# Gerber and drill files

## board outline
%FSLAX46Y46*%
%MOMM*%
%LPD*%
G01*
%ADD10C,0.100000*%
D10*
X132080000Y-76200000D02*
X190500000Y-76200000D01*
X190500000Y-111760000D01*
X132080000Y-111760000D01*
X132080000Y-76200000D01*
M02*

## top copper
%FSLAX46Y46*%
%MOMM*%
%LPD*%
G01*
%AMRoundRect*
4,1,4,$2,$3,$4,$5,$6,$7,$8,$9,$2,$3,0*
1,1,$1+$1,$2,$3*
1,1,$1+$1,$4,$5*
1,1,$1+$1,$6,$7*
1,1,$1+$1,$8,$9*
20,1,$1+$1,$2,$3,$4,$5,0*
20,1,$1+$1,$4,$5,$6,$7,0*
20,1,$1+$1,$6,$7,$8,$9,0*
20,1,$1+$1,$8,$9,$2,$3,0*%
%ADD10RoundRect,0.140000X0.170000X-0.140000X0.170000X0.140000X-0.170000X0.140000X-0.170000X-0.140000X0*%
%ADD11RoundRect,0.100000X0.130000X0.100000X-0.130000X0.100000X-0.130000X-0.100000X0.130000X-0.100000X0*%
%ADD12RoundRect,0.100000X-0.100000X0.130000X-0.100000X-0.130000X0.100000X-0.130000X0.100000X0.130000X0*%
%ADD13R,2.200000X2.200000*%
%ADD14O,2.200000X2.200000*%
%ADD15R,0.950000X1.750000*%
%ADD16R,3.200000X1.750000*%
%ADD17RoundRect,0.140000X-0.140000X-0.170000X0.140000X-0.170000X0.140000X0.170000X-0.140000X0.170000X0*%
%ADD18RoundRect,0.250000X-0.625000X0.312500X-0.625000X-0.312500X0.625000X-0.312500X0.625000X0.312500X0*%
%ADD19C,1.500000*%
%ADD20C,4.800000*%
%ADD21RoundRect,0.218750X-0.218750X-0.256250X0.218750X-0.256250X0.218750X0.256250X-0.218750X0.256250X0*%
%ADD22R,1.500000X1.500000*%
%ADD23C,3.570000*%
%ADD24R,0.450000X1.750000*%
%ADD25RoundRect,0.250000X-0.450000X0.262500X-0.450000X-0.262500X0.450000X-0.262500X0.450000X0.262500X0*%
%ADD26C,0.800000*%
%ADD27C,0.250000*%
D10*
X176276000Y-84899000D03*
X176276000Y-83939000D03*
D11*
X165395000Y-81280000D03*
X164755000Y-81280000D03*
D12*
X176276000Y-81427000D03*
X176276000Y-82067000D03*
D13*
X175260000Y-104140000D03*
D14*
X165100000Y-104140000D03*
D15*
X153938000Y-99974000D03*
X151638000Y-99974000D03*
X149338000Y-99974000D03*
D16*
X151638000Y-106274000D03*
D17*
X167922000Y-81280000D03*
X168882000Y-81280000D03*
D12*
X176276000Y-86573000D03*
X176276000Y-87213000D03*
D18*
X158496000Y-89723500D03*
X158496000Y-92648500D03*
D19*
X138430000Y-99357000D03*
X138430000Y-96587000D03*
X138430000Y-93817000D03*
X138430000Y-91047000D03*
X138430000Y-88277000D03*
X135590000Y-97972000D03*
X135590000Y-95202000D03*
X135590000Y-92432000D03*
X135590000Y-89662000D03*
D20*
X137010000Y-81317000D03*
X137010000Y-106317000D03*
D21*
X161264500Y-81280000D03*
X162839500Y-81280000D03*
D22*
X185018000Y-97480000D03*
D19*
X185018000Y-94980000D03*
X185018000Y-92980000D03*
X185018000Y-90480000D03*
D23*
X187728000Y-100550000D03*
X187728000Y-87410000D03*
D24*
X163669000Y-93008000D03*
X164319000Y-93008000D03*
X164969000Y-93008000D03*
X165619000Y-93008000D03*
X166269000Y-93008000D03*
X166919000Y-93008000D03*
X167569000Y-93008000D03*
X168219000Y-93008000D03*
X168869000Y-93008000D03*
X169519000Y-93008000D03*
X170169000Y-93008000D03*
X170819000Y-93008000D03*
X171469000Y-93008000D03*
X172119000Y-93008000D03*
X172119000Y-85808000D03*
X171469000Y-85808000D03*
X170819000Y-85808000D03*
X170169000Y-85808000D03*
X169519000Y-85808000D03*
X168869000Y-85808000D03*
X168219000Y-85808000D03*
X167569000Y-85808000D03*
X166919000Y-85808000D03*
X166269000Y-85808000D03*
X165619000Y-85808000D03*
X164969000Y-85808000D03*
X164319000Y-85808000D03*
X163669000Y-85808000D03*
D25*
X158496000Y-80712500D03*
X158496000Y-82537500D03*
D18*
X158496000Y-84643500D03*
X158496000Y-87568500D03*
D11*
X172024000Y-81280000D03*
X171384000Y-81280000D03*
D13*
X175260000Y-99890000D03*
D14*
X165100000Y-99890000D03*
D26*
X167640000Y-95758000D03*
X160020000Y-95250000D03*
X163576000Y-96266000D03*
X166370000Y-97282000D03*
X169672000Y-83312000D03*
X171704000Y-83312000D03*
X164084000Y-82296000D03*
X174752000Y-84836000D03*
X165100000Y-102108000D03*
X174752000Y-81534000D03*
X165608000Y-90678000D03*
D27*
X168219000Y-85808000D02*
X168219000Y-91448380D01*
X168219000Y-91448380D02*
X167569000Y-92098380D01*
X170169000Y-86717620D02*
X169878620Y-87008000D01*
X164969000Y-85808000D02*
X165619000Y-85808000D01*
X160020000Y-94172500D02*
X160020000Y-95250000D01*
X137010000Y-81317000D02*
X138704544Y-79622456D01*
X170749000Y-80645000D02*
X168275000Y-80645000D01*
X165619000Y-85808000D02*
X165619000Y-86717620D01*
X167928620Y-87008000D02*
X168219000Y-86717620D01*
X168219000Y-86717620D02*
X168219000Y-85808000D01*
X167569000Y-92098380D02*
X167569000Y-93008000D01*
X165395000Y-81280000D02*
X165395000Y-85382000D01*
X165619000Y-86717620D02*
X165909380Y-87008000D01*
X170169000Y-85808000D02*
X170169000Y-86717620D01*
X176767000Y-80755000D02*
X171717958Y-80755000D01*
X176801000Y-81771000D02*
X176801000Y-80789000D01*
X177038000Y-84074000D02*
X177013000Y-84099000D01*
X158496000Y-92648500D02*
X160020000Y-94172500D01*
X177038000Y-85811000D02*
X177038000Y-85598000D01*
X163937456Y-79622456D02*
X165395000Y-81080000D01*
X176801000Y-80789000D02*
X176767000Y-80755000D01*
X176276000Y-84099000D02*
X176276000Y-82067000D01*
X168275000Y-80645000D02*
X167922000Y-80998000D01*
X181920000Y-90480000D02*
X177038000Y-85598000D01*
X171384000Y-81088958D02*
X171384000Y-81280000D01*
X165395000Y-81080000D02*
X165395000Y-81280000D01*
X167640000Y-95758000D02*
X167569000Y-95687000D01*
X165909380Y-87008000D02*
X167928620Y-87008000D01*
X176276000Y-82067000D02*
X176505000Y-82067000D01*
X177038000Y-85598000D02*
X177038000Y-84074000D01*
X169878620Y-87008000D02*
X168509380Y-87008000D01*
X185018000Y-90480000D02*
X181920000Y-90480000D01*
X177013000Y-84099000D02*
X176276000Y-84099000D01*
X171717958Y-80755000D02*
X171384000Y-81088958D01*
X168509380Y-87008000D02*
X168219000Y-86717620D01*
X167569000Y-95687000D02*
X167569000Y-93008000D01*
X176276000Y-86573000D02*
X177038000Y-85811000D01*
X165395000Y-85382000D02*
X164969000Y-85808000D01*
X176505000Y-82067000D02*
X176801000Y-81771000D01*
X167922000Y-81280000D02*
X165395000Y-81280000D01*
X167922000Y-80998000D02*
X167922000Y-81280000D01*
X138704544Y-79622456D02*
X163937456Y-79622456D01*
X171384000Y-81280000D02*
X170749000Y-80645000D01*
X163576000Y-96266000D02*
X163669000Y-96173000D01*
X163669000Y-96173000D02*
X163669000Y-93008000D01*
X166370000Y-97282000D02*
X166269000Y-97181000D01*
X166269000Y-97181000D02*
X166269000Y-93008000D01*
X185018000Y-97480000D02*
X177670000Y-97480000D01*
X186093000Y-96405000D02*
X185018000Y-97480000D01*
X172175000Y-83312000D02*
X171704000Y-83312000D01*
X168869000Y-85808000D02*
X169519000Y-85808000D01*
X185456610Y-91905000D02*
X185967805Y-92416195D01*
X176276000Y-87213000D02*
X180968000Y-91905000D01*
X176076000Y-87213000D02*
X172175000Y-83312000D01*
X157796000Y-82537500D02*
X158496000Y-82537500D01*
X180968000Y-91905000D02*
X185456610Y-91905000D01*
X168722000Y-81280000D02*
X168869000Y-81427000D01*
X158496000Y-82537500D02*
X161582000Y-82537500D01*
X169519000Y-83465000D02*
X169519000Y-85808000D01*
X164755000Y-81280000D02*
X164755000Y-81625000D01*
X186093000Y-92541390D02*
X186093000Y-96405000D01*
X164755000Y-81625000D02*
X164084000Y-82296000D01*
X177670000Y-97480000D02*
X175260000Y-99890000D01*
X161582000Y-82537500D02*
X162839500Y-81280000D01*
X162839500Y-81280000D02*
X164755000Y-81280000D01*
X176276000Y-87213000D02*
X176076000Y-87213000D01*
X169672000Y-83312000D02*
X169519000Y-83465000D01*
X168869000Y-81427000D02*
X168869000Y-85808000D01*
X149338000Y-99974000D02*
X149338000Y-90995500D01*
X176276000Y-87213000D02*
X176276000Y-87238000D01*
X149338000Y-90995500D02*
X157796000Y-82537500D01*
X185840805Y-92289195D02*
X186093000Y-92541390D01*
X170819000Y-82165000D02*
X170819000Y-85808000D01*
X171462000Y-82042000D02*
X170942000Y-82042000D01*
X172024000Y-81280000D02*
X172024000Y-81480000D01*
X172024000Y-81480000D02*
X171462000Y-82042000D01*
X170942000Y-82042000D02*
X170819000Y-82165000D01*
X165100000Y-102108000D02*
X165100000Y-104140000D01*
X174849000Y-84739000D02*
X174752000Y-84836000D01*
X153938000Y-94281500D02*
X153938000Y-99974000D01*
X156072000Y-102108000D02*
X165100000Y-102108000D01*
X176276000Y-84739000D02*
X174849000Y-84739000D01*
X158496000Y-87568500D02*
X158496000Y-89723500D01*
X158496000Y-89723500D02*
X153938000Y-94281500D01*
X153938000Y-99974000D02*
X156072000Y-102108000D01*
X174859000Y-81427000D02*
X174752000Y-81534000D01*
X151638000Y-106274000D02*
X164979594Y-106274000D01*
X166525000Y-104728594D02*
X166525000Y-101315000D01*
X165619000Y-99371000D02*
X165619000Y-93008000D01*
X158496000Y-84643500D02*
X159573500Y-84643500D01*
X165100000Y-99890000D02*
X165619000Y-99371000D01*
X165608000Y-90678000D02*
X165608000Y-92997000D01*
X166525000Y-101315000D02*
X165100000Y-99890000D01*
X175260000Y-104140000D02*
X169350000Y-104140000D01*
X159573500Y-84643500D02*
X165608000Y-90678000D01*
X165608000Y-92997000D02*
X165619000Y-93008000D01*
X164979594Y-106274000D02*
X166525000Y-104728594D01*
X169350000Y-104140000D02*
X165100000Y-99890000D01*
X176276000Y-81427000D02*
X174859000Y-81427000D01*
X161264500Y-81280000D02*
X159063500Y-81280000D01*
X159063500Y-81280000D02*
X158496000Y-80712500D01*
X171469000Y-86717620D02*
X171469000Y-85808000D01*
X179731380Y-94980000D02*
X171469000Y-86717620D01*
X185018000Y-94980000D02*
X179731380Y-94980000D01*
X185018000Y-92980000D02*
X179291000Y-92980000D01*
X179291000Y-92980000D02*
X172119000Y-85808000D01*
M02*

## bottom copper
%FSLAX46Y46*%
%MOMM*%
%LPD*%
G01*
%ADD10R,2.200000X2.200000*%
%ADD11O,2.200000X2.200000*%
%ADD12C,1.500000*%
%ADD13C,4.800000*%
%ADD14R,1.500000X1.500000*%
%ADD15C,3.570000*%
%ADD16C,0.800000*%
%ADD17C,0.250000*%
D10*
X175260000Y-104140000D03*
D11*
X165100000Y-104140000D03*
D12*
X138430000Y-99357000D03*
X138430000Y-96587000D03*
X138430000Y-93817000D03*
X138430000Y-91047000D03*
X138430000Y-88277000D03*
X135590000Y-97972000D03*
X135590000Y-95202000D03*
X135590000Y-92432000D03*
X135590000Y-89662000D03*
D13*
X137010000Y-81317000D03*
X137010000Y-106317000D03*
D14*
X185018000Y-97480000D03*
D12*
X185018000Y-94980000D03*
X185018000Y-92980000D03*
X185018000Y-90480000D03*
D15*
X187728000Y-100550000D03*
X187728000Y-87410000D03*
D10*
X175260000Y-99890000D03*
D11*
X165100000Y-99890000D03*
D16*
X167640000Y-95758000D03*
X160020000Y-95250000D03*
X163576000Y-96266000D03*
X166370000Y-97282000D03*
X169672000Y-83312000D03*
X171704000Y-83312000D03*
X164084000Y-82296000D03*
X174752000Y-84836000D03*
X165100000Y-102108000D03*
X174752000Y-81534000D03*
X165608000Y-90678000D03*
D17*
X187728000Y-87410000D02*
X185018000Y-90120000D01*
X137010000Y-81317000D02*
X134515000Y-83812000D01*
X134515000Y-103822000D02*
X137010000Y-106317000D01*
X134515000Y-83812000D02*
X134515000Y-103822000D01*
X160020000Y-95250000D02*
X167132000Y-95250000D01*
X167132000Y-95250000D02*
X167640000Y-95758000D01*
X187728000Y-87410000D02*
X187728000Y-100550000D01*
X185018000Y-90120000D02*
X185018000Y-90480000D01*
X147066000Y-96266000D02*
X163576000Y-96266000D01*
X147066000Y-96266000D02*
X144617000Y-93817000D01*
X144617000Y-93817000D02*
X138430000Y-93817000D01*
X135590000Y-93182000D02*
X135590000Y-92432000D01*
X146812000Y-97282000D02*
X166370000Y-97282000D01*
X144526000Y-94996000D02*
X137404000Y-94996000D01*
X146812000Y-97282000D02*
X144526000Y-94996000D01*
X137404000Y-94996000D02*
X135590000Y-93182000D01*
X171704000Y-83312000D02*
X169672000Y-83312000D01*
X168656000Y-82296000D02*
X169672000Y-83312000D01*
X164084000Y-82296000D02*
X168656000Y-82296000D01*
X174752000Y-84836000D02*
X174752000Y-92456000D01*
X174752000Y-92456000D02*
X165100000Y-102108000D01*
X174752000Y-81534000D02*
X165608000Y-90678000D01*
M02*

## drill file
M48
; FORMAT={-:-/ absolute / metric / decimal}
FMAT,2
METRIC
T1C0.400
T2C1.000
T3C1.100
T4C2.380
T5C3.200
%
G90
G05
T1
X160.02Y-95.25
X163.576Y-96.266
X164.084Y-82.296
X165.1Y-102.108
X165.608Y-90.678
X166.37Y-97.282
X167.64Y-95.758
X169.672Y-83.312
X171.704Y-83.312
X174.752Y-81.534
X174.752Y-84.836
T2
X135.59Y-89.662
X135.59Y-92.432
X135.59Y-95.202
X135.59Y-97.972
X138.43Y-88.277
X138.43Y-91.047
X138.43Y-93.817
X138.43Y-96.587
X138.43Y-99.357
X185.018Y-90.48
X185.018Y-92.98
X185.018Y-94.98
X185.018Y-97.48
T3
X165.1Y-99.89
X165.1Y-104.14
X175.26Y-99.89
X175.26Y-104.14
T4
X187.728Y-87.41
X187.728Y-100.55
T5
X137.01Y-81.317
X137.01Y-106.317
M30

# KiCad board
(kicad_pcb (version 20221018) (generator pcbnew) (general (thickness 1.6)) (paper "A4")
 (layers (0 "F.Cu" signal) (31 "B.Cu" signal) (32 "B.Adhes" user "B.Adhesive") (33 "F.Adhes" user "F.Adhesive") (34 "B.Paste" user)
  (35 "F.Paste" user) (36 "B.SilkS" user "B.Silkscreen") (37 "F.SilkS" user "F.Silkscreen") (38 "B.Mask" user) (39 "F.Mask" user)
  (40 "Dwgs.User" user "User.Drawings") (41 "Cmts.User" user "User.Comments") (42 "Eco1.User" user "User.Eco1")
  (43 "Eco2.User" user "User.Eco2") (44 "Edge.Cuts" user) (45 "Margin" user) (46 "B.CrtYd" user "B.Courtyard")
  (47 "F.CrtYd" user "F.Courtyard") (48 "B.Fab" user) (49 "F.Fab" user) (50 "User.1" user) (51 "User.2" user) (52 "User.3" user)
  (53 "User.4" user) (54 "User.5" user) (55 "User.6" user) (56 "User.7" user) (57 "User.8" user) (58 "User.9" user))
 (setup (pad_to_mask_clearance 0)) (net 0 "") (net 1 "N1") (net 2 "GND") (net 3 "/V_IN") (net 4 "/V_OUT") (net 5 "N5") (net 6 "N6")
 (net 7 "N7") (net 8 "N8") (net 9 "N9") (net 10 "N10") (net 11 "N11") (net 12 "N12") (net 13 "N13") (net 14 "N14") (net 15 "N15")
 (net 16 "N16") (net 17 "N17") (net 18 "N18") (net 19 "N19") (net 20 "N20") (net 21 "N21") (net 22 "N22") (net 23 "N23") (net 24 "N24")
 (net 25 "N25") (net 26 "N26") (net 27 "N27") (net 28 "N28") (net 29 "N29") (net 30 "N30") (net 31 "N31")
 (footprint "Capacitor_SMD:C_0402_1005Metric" (layer "F.Cu") (at 176.276 84.419 90)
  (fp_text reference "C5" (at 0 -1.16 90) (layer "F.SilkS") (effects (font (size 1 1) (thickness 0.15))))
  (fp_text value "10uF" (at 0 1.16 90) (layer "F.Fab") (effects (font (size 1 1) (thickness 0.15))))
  (pad "1" smd roundrect (at -0.48 0 90) (size 0.56 0.62) (layers "F.Cu" "F.Paste" "F.Mask") (roundrect_rratio 0.25) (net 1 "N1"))
  (pad "2" smd roundrect (at 0.48 0 90) (size 0.56 0.62) (layers "F.Cu" "F.Paste" "F.Mask") (roundrect_rratio 0.25) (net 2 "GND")))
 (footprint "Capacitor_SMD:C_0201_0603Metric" (layer "F.Cu") (at 165.075 81.28 180)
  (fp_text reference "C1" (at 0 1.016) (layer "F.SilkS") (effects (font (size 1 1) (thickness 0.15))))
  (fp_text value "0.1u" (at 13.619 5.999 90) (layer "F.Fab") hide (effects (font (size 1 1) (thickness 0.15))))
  (pad "" smd roundrect (at -0.345 0 180) (size 0.318 0.36) (layers "F.Paste") (roundrect_rratio 0.25))
  (pad "" smd roundrect (at 0.345 0 180) (size 0.318 0.36) (layers "F.Paste") (roundrect_rratio 0.25))
  (pad "1" smd roundrect (at -0.32 0 180) (size 0.46 0.4) (layers "F.Cu" "F.Mask") (roundrect_rratio 0.25) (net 2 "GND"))
  (pad "2" smd roundrect (at 0.32 0 180) (size 0.46 0.4) (layers "F.Cu" "F.Mask") (roundrect_rratio 0.25) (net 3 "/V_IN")))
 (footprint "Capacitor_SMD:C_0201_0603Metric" (layer "F.Cu") (at 176.276 81.747 -90)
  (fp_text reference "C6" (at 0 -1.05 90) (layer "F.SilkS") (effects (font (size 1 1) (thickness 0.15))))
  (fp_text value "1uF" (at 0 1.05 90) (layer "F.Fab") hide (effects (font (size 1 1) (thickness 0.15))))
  (pad "" smd roundrect (at -0.345 0 270) (size 0.318 0.36) (layers "F.Paste") (roundrect_rratio 0.25))
  (pad "" smd roundrect (at 0.345 0 270) (size 0.318 0.36) (layers "F.Paste") (roundrect_rratio 0.25))
  (pad "1" smd roundrect (at -0.32 0 270) (size 0.46 0.4) (layers "F.Cu" "F.Mask") (roundrect_rratio 0.25) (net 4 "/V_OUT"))
  (pad "2" smd roundrect (at 0.32 0 270) (size 0.46 0.4) (layers "F.Cu" "F.Mask") (roundrect_rratio 0.25) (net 2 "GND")))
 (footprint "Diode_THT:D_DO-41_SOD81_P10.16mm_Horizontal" (layer "F.Cu") (at 175.26 104.14 180)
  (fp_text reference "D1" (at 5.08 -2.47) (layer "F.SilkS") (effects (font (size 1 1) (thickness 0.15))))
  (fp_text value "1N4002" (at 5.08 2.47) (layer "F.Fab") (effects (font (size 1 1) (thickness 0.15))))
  (pad "1" thru_hole rect (at 0 0 180) (size 2.2 2.2) (drill 1.1) (layers "*.Cu" "*.Mask") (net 4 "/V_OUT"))
  (pad "2" thru_hole oval (at 10.16 0 180) (size 2.2 2.2) (drill 1.1) (layers "*.Cu" "*.Mask") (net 1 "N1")))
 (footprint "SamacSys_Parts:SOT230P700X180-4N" (layer "F.Cu") (at 151.638 103.124 -90)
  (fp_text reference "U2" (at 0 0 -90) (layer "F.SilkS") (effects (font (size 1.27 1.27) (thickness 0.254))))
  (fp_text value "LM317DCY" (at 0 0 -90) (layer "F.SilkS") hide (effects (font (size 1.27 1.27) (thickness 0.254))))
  (pad "1" smd rect (at -3.15 -2.3) (size 0.95 1.75) (layers "F.Cu" "F.Paste" "F.Mask") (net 1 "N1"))
  (pad "2" smd rect (at -3.15 0) (size 0.95 1.75) (layers "F.Cu" "F.Paste" "F.Mask") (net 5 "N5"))
  (pad "3" smd rect (at -3.15 2.3) (size 0.95 1.75) (layers "F.Cu" "F.Paste" "F.Mask") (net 3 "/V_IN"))
  (pad "4" smd rect (at 3.15 0 270) (size 1.75 3.2) (layers "F.Cu" "F.Paste" "F.Mask") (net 4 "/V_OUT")))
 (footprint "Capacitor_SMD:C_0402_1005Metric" (layer "F.Cu") (at 168.402 81.28)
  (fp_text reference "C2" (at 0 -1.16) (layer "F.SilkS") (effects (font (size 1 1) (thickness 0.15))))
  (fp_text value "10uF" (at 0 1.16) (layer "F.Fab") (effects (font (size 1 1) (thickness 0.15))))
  (pad "1" smd roundrect (at -0.48 0) (size 0.56 0.62) (layers "F.Cu" "F.Paste" "F.Mask") (roundrect_rratio 0.25) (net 2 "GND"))
  (pad "2" smd roundrect (at 0.48 0) (size 0.56 0.62) (layers "F.Cu" "F.Paste" "F.Mask") (roundrect_rratio 0.25) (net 3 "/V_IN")))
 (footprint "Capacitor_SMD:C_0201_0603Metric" (layer "F.Cu") (at 176.276 86.893 -90)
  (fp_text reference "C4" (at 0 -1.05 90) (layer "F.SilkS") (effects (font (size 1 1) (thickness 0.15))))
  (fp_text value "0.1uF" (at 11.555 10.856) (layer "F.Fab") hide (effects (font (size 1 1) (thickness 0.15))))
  (pad "" smd roundrect (at -0.345 0 270) (size 0.318 0.36) (layers "F.Paste") (roundrect_rratio 0.25))
  (pad "" smd roundrect (at 0.345 0 270) (size 0.318 0.36) (layers "F.Paste") (roundrect_rratio 0.25))
  (pad "1" smd roundrect (at -0.32 0 270) (size 0.46 0.4) (layers "F.Cu" "F.Mask") (roundrect_rratio 0.25) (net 2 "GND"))
  (pad "2" smd roundrect (at 0.32 0 270) (size 0.46 0.4) (layers "F.Cu" "F.Mask") (roundrect_rratio 0.25) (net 3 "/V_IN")))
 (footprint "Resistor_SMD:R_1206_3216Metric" (layer "F.Cu") (at 158.496 91.186 -90)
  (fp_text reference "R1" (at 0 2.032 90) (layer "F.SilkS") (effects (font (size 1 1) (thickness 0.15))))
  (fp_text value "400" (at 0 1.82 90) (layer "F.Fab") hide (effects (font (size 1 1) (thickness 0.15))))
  (pad "1" smd roundrect (at -1.4625 0 270) (size 1.125 1.75) (layers "F.Cu" "F.Paste" "F.Mask") (roundrect_rratio 0.2222222222)
   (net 1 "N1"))
  (pad "2" smd roundrect (at 1.4625 0 270) (size 1.125 1.75) (layers "F.Cu" "F.Paste" "F.Mask") (roundrect_rratio 0.2222222222)
   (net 2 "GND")))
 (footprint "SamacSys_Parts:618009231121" (layer "F.Cu") (at 138.43 99.357 -90)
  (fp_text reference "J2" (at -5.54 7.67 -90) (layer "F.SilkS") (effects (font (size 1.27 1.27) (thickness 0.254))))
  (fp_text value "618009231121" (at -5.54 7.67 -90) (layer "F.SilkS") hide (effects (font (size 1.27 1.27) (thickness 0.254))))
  (pad "1" thru_hole circle (at 0 0 270) (size 1.5 1.5) (drill 1) (layers "*.Cu" "*.Mask") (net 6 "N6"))
  (pad "2" thru_hole circle (at -2.77 0 270) (size 1.5 1.5) (drill 1) (layers "*.Cu" "*.Mask") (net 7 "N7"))
  (pad "3" thru_hole circle (at -5.54 0 270) (size 1.5 1.5) (drill 1) (layers "*.Cu" "*.Mask") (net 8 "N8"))
  (pad "4" thru_hole circle (at -8.31 0 270) (size 1.5 1.5) (drill 1) (layers "*.Cu" "*.Mask") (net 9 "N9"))
  (pad "5" thru_hole circle (at -11.08 0 270) (size 1.5 1.5) (drill 1) (layers "*.Cu" "*.Mask") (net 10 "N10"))
  (pad "6" thru_hole circle (at -1.385 2.84 270) (size 1.5 1.5) (drill 1) (layers "*.Cu" "*.Mask") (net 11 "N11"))
  (pad "7" thru_hole circle (at -4.155 2.84 270) (size 1.5 1.5) (drill 1) (layers "*.Cu" "*.Mask") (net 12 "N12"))
  (pad "8" thru_hole circle (at -6.925 2.84 270) (size 1.5 1.5) (drill 1) (layers "*.Cu" "*.Mask") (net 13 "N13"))
  (pad "9" thru_hole circle (at -9.695 2.84 270) (size 1.5 1.5) (drill 1) (layers "*.Cu" "*.Mask") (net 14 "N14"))
  (pad "MH1" thru_hole circle (at -18.04 1.42 270) (size 4.8 4.8) (drill 3.2) (layers "*.Cu" "*.Mask") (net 2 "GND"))
  (pad "MH2" thru_hole circle (at 6.96 1.42 270) (size 4.8 4.8) (drill 3.2) (layers "*.Cu" "*.Mask") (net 2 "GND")))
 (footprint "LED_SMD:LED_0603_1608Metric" (layer "F.Cu") (at 162.052 81.28)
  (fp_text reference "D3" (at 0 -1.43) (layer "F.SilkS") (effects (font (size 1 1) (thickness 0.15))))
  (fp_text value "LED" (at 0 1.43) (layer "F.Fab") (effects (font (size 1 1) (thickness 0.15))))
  (pad "1" smd roundrect (at -0.7875 0) (size 0.875 0.95) (layers "F.Cu" "F.Paste" "F.Mask") (roundrect_rratio 0.25) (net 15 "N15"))
  (pad "2" smd roundrect (at 0.7875 0) (size 0.875 0.95) (layers "F.Cu" "F.Paste" "F.Mask") (roundrect_rratio 0.25) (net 3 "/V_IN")))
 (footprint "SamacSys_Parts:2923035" (layer "F.Cu") (at 185.018 97.48 90)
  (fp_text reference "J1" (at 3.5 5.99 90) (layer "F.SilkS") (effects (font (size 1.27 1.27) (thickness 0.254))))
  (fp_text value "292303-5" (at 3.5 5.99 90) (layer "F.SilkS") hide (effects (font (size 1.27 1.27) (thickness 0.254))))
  (pad "1" thru_hole rect (at 0 0 90) (size 1.5 1.5) (drill 1) (layers "*.Cu" "*.Mask") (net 3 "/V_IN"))
  (pad "2" thru_hole circle (at 2.5 0 90) (size 1.5 1.5) (drill 1) (layers "*.Cu" "*.Mask") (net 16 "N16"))
  (pad "3" thru_hole circle (at 4.5 0 90) (size 1.5 1.5) (drill 1) (layers "*.Cu" "*.Mask") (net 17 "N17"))
  (pad "4" thru_hole circle (at 7 0 90) (size 1.5 1.5) (drill 1) (layers "*.Cu" "*.Mask") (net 2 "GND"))
  (pad "MH1" thru_hole circle (at -3.07 2.71 90) (size 3.57 3.57) (drill 2.38) (layers "*.Cu" "*.Mask") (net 2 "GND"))
  (pad "MH2" thru_hole circle (at 10.07 2.71 90) (size 3.57 3.57) (drill 2.38) (layers "*.Cu" "*.Mask") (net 2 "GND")))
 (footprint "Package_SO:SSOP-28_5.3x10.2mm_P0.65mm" (layer "F.Cu") (at 167.894 89.408 90)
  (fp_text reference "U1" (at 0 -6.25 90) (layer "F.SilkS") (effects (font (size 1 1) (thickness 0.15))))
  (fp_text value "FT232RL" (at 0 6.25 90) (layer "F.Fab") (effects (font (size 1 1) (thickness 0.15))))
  (pad "1" smd rect (at -3.6 -4.225 90) (size 1.75 0.45) (layers "F.Cu" "F.Paste" "F.Mask") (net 8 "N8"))
  (pad "2" smd rect (at -3.6 -3.575 90) (size 1.75 0.45) (layers "F.Cu" "F.Paste" "F.Mask") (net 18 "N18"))
  (pad "3" smd rect (at -3.6 -2.925 90) (size 1.75 0.45) (layers "F.Cu" "F.Paste" "F.Mask") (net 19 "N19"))
  (pad "4" smd rect (at -3.6 -2.275 90) (size 1.75 0.45) (layers "F.Cu" "F.Paste" "F.Mask") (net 4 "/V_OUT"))
  (pad "5" smd rect (at -3.6 -1.625 90) (size 1.75 0.45) (layers "F.Cu" "F.Paste" "F.Mask") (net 13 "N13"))
  (pad "6" smd rect (at -3.6 -0.975 90) (size 1.75 0.45) (layers "F.Cu" "F.Paste" "F.Mask") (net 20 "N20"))
  (pad "7" smd rect (at -3.6 -0.325 90) (size 1.75 0.45) (layers "F.Cu" "F.Paste" "F.Mask") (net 2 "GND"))
  (pad "8" smd rect (at -3.6 0.325 90) (size 1.75 0.45) (layers "F.Cu" "F.Paste" "F.Mask"))
  (pad "9" smd rect (at -3.6 0.975 90) (size 1.75 0.45) (layers "F.Cu" "F.Paste" "F.Mask") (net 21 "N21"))
  (pad "10" smd rect (at -3.6 1.625 90) (size 1.75 0.45) (layers "F.Cu" "F.Paste" "F.Mask") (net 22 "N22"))
  (pad "11" smd rect (at -3.6 2.275 90) (size 1.75 0.45) (layers "F.Cu" "F.Paste" "F.Mask") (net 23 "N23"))
  (pad "12" smd rect (at -3.6 2.925 90) (size 1.75 0.45) (layers "F.Cu" "F.Paste" "F.Mask") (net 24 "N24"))
  (pad "13" smd rect (at -3.6 3.575 90) (size 1.75 0.45) (layers "F.Cu" "F.Paste" "F.Mask") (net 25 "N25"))
  (pad "14" smd rect (at -3.6 4.225 90) (size 1.75 0.45) (layers "F.Cu" "F.Paste" "F.Mask") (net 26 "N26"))
  (pad "15" smd rect (at 3.6 4.225 90) (size 1.75 0.45) (layers "F.Cu" "F.Paste" "F.Mask") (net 17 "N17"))
  (pad "16" smd rect (at 3.6 3.575 90) (size 1.75 0.45) (layers "F.Cu" "F.Paste" "F.Mask") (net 16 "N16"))
  (pad "17" smd rect (at 3.6 2.925 90) (size 1.75 0.45) (layers "F.Cu" "F.Paste" "F.Mask") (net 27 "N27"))
  (pad "18" smd rect (at 3.6 2.275 90) (size 1.75 0.45) (layers "F.Cu" "F.Paste" "F.Mask") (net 2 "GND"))
  (pad "19" smd rect (at 3.6 1.625 90) (size 1.75 0.45) (layers "F.Cu" "F.Paste" "F.Mask") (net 3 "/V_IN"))
  (pad "20" smd rect (at 3.6 0.975 90) (size 1.75 0.45) (layers "F.Cu" "F.Paste" "F.Mask") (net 3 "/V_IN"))
  (pad "21" smd rect (at 3.6 0.325 90) (size 1.75 0.45) (layers "F.Cu" "F.Paste" "F.Mask") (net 2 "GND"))
  (pad "22" smd rect (at 3.6 -0.325 90) (size 1.75 0.45) (layers "F.Cu" "F.Paste" "F.Mask") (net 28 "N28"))
  (pad "23" smd rect (at 3.6 -0.975 90) (size 1.75 0.45) (layers "F.Cu" "F.Paste" "F.Mask") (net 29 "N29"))
  (pad "24" smd rect (at 3.6 -1.625 90) (size 1.75 0.45) (layers "F.Cu" "F.Paste" "F.Mask"))
  (pad "25" smd rect (at 3.6 -2.275 90) (size 1.75 0.45) (layers "F.Cu" "F.Paste" "F.Mask") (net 2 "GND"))
  (pad "26" smd rect (at 3.6 -2.925 90) (size 1.75 0.45) (layers "F.Cu" "F.Paste" "F.Mask") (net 2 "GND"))
  (pad "27" smd rect (at 3.6 -3.575 90) (size 1.75 0.45) (layers "F.Cu" "F.Paste" "F.Mask") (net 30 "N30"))
  (pad "28" smd rect (at 3.6 -4.225 90) (size 1.75 0.45) (layers "F.Cu" "F.Paste" "F.Mask") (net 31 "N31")))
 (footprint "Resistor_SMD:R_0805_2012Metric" (layer "F.Cu") (at 158.496 81.625 -90)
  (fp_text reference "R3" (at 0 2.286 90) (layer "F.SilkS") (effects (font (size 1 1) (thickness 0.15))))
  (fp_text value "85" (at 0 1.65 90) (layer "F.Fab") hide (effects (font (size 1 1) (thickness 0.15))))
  (pad "1" smd roundrect (at -0.9125 0 270) (size 1.025 1.4) (layers "F.Cu" "F.Paste" "F.Mask") (roundrect_rratio 0.243902439)
   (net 15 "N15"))
  (pad "2" smd roundrect (at 0.9125 0 270) (size 1.025 1.4) (layers "F.Cu" "F.Paste" "F.Mask") (roundrect_rratio 0.243902439)
   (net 3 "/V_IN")))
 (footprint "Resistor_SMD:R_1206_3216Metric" (layer "F.Cu") (at 158.496 86.106 -90)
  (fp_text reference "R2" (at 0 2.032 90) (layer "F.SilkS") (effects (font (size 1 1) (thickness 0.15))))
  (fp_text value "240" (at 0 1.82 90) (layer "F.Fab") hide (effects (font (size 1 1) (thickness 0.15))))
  (pad "1" smd roundrect (at -1.4625 0 270) (size 1.125 1.75) (layers "F.Cu" "F.Paste" "F.Mask") (roundrect_rratio 0.2222222222)
   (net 4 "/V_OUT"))
  (pad "2" smd roundrect (at 1.4625 0 270) (size 1.125 1.75) (layers "F.Cu" "F.Paste" "F.Mask") (roundrect_rratio 0.2222222222) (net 1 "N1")))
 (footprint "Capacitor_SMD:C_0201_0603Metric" (layer "F.Cu") (at 171.704 81.28 180)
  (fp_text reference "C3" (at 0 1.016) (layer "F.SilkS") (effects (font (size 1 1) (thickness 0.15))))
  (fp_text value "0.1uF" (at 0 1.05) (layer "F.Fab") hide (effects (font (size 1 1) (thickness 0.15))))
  (pad "" smd roundrect (at -0.345 0 180) (size 0.318 0.36) (layers "F.Paste") (roundrect_rratio 0.25))
  (pad "" smd roundrect (at 0.345 0 180) (size 0.318 0.36) (layers "F.Paste") (roundrect_rratio 0.25))
  (pad "1" smd roundrect (at -0.32 0 180) (size 0.46 0.4) (layers "F.Cu" "F.Mask") (roundrect_rratio 0.25) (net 27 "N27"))
  (pad "2" smd roundrect (at 0.32 0 180) (size 0.46 0.4) (layers "F.Cu" "F.Mask") (roundrect_rratio 0.25) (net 2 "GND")))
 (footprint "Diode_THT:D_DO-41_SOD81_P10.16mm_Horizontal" (layer "F.Cu") (at 175.26 99.89 180)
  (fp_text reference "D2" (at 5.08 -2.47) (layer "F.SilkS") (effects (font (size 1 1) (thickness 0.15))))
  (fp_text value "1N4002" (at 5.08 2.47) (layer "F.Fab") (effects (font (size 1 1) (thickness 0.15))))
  (pad "1" thru_hole rect (at 0 0 180) (size 2.2 2.2) (drill 1.1) (layers "*.Cu" "*.Mask") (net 3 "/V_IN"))
  (pad "2" thru_hole oval (at 10.16 0 180) (size 2.2 2.2) (drill 1.1) (layers "*.Cu" "*.Mask") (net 4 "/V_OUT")))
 (gr_rect (start 132.08 76.2) (end 190.5 111.76) (stroke (width 0.1) (type default)) (fill none) (layer "Edge.Cuts"))
 (segment (start 168.219 85.808) (end 168.219 91.44838) (width 0.25) (layer "F.Cu") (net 2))
 (segment (start 168.219 91.44838) (end 167.569 92.09838) (width 0.25) (layer "F.Cu") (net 2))
 (segment (start 170.169 86.71762) (end 169.87862 87.008) (width 0.25) (layer "F.Cu") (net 2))
 (segment (start 164.969 85.808) (end 165.619 85.808) (width 0.25) (layer "F.Cu") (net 2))
 (segment (start 160.02 94.1725) (end 160.02 95.25) (width 0.25) (layer "F.Cu") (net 2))
 (segment (start 137.01 81.317) (end 138.704544 79.622456) (width 0.25) (layer "F.Cu") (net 2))
 (segment (start 170.749 80.645) (end 168.275 80.645) (width 0.25) (layer "F.Cu") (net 2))
 (segment (start 165.619 85.808) (end 165.619 86.71762) (width 0.25) (layer "F.Cu") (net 2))
 (segment (start 167.92862 87.008) (end 168.219 86.71762) (width 0.25) (layer "F.Cu") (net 2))
 (segment (start 168.219 86.71762) (end 168.219 85.808) (width 0.25) (layer "F.Cu") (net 2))
 (segment (start 167.569 92.09838) (end 167.569 93.008) (width 0.25) (layer "F.Cu") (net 2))
 (segment (start 165.395 81.28) (end 165.395 85.382) (width 0.25) (layer "F.Cu") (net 2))
 (segment (start 165.619 86.71762) (end 165.90938 87.008) (width 0.25) (layer "F.Cu") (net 2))
 (segment (start 170.169 85.808) (end 170.169 86.71762) (width 0.25) (layer "F.Cu") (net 2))
 (segment (start 176.767 80.755) (end 171.717958 80.755) (width 0.25) (layer "F.Cu") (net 2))
 (segment (start 176.801 81.771) (end 176.801 80.789) (width 0.25) (layer "F.Cu") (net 2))
 (segment (start 177.038 84.074) (end 177.013 84.099) (width 0.25) (layer "F.Cu") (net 2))
 (segment (start 158.496 92.6485) (end 160.02 94.1725) (width 0.25) (layer "F.Cu") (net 2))
 (segment (start 177.038 85.811) (end 177.038 85.598) (width 0.25) (layer "F.Cu") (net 2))
 (segment (start 163.937456 79.622456) (end 165.395 81.08) (width 0.25) (layer "F.Cu") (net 2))
 (segment (start 176.801 80.789) (end 176.767 80.755) (width 0.25) (layer "F.Cu") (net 2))
 (segment (start 176.276 84.099) (end 176.276 82.067) (width 0.25) (layer "F.Cu") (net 2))
 (segment (start 168.275 80.645) (end 167.922 80.998) (width 0.25) (layer "F.Cu") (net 2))
 (segment (start 181.92 90.48) (end 177.038 85.598) (width 0.25) (layer "F.Cu") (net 2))
 (segment (start 171.384 81.088958) (end 171.384 81.28) (width 0.25) (layer "F.Cu") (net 2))
 (segment (start 165.395 81.08) (end 165.395 81.28) (width 0.25) (layer "F.Cu") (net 2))
 (segment (start 167.64 95.758) (end 167.569 95.687) (width 0.25) (layer "F.Cu") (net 2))
 (segment (start 165.90938 87.008) (end 167.92862 87.008) (width 0.25) (layer "F.Cu") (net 2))
 (segment (start 176.276 82.067) (end 176.505 82.067) (width 0.25) (layer "F.Cu") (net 2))
 (segment (start 177.038 85.598) (end 177.038 84.074) (width 0.25) (layer "F.Cu") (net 2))
 (segment (start 169.87862 87.008) (end 168.50938 87.008) (width 0.25) (layer "F.Cu") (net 2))
 (segment (start 185.018 90.48) (end 181.92 90.48) (width 0.25) (layer "F.Cu") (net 2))
 (segment (start 177.013 84.099) (end 176.276 84.099) (width 0.25) (layer "F.Cu") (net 2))
 (segment (start 171.717958 80.755) (end 171.384 81.088958) (width 0.25) (layer "F.Cu") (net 2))
 (segment (start 168.50938 87.008) (end 168.219 86.71762) (width 0.25) (layer "F.Cu") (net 2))
 (segment (start 167.569 95.687) (end 167.569 93.008) (width 0.25) (layer "F.Cu") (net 2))
 (segment (start 176.276 86.573) (end 177.038 85.811) (width 0.25) (layer "F.Cu") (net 2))
 (segment (start 165.395 85.382) (end 164.969 85.808) (width 0.25) (layer "F.Cu") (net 2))
 (segment (start 176.505 82.067) (end 176.801 81.771) (width 0.25) (layer "F.Cu") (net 2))
 (segment (start 167.922 81.28) (end 165.395 81.28) (width 0.25) (layer "F.Cu") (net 2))
 (segment (start 167.922 80.998) (end 167.922 81.28) (width 0.25) (layer "F.Cu") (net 2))
 (segment (start 138.704544 79.622456) (end 163.937456 79.622456) (width 0.25) (layer "F.Cu") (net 2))
 (segment (start 171.384 81.28) (end 170.749 80.645) (width 0.25) (layer "F.Cu") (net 2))
 (via (at 167.64 95.758) (size 0.8) (drill 0.4) (layers "F.Cu" "B.Cu") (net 2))
 (via (at 160.02 95.25) (size 0.8) (drill 0.4) (layers "F.Cu" "B.Cu") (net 2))
 (segment (start 187.728 87.41) (end 185.018 90.12) (width 0.25) (layer "B.Cu") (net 2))
 (segment (start 137.01 81.317) (end 134.515 83.812) (width 0.25) (layer "B.Cu") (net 2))
 (segment (start 134.515 103.822) (end 137.01 106.317) (width 0.25) (layer "B.Cu") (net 2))
 (segment (start 134.515 83.812) (end 134.515 103.822) (width 0.25) (layer "B.Cu") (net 2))
 (segment (start 160.02 95.25) (end 167.132 95.25) (width 0.25) (layer "B.Cu") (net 2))
 (segment (start 167.132 95.25) (end 167.64 95.758) (width 0.25) (layer "B.Cu") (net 2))
 (segment (start 187.728 87.41) (end 187.728 100.55) (width 0.25) (layer "B.Cu") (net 2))
 (segment (start 185.018 90.12) (end 185.018 90.48) (width 0.25) (layer "B.Cu") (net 2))
 (segment (start 163.576 96.266) (end 163.669 96.173) (width 0.25) (layer "F.Cu") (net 8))
 (segment (start 163.669 96.173) (end 163.669 93.008) (width 0.25) (layer "F.Cu") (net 8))
 (via (at 163.576 96.266) (size 0.8) (drill 0.4) (layers "F.Cu" "B.Cu") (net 8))
 (segment (start 147.066 96.266) (end 163.576 96.266) (width 0.25) (layer "B.Cu") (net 8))
 (segment (start 147.066 96.266) (end 144.617 93.817) (width 0.25) (layer "B.Cu") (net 8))
 (segment (start 144.617 93.817) (end 138.43 93.817) (width 0.25) (layer "B.Cu") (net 8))
 (segment (start 166.37 97.282) (end 166.269 97.181) (width 0.25) (layer "F.Cu") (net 13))
 (segment (start 166.269 97.181) (end 166.269 93.008) (width 0.25) (layer "F.Cu") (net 13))
 (via (at 166.37 97.282) (size 0.8) (drill 0.4) (layers "F.Cu" "B.Cu") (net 13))
 (segment (start 135.59 93.182) (end 135.59 92.432) (width 0.25) (layer "B.Cu") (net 13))
 (segment (start 146.812 97.282) (end 166.37 97.282) (width 0.25) (layer "B.Cu") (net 13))
 (segment (start 144.526 94.996) (end 137.404 94.996) (width 0.25) (layer "B.Cu") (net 13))
 (segment (start 146.812 97.282) (end 144.526 94.996) (width 0.25) (layer "B.Cu") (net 13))
 (segment (start 137.404 94.996) (end 135.59 93.182) (width 0.25) (layer "B.Cu") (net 13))
 (segment (start 185.018 97.48) (end 177.67 97.48) (width 0.25) (layer "F.Cu") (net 3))
 (segment (start 186.093 96.405) (end 185.018 97.48) (width 0.25) (layer "F.Cu") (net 3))
 (segment (start 172.175 83.312) (end 171.704 83.312) (width 0.25) (layer "F.Cu") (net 3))
 (segment (start 168.869 85.808) (end 169.519 85.808) (width 0.25) (layer "F.Cu") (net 3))
 (segment (start 185.45661 91.905) (end 185.967805 92.416195) (width 0.25) (layer "F.Cu") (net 3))
 (segment (start 176.276 87.213) (end 180.968 91.905) (width 0.25) (layer "F.Cu") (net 3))
 (segment (start 176.076 87.213) (end 172.175 83.312) (width 0.25) (layer "F.Cu") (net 3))
 (segment (start 157.796 82.5375) (end 158.496 82.5375) (width 0.25) (layer "F.Cu") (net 3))
 (segment (start 180.968 91.905) (end 185.45661 91.905) (width 0.25) (layer "F.Cu") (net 3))
 (segment (start 168.722 81.28) (end 168.869 81.427) (width 0.25) (layer "F.Cu") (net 3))
 (segment (start 158.496 82.5375) (end 161.582 82.5375) (width 0.25) (layer "F.Cu") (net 3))
 (segment (start 169.519 83.465) (end 169.519 85.808) (width 0.25) (layer "F.Cu") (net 3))
 (segment (start 164.755 81.28) (end 164.755 81.625) (width 0.25) (layer "F.Cu") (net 3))
 (segment (start 186.093 92.54139) (end 186.093 96.405) (width 0.25) (layer "F.Cu") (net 3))
 (segment (start 164.755 81.625) (end 164.084 82.296) (width 0.25) (layer "F.Cu") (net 3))
 (segment (start 177.67 97.48) (end 175.26 99.89) (width 0.25) (layer "F.Cu") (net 3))
 (segment (start 161.582 82.5375) (end 162.8395 81.28) (width 0.25) (layer "F.Cu") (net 3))
 (segment (start 162.8395 81.28) (end 164.755 81.28) (width 0.25) (layer "F.Cu") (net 3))
 (segment (start 176.276 87.213) (end 176.076 87.213) (width 0.25) (layer "F.Cu") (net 3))
 (segment (start 169.672 83.312) (end 169.519 83.465) (width 0.25) (layer "F.Cu") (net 3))
 (segment (start 168.869 81.427) (end 168.869 85.808) (width 0.25) (layer "F.Cu") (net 3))
 (segment (start 149.338 99.974) (end 149.338 90.9955) (width 0.25) (layer "F.Cu") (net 3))
 (segment (start 176.276 87.213) (end 176.276 87.238) (width 0.25) (layer "F.Cu") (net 3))
 (segment (start 149.338 90.9955) (end 157.796 82.5375) (width 0.25) (layer "F.Cu") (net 3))
 (segment (start 185.840805 92.289195) (end 186.093 92.54139) (width 0.25) (layer "F.Cu") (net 3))
 (via (at 169.672 83.312) (size 0.8) (drill 0.4) (layers "F.Cu" "B.Cu") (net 3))
 (via (at 171.704 83.312) (size 0.8) (drill 0.4) (layers "F.Cu" "B.Cu") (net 3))
 (via (at 164.084 82.296) (size 0.8) (drill 0.4) (layers "F.Cu" "B.Cu") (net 3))
 (segment (start 171.704 83.312) (end 169.672 83.312) (width 0.25) (layer "B.Cu") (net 3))
 (segment (start 168.656 82.296) (end 169.672 83.312) (width 0.25) (layer "B.Cu") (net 3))
 (segment (start 164.084 82.296) (end 168.656 82.296) (width 0.25) (layer "B.Cu") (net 3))
 (segment (start 170.819 82.165) (end 170.819 85.808) (width 0.25) (layer "F.Cu") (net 27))
 (segment (start 171.462 82.042) (end 170.942 82.042) (width 0.25) (layer "F.Cu") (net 27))
 (segment (start 172.024 81.28) (end 172.024 81.48) (width 0.25) (layer "F.Cu") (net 27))
 (segment (start 172.024 81.48) (end 171.462 82.042) (width 0.25) (layer "F.Cu") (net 27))
 (segment (start 170.942 82.042) (end 170.819 82.165) (width 0.25) (layer "F.Cu") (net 27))
 (segment (start 165.1 102.108) (end 165.1 104.14) (width 0.25) (layer "F.Cu") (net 1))
 (segment (start 174.849 84.739) (end 174.752 84.836) (width 0.25) (layer "F.Cu") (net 1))
 (segment (start 153.938 94.2815) (end 153.938 99.974) (width 0.25) (layer "F.Cu") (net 1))
 (segment (start 156.072 102.108) (end 165.1 102.108) (width 0.25) (layer "F.Cu") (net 1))
 (segment (start 176.276 84.739) (end 174.849 84.739) (width 0.25) (layer "F.Cu") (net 1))
 (segment (start 158.496 87.5685) (end 158.496 89.7235) (width 0.25) (layer "F.Cu") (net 1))
 (segment (start 158.496 89.7235) (end 153.938 94.2815) (width 0.25) (layer "F.Cu") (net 1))
 (segment (start 153.938 99.974) (end 156.072 102.108) (width 0.25) (layer "F.Cu") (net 1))
 (via (at 174.752 84.836) (size 0.8) (drill 0.4) (layers "F.Cu" "B.Cu") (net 1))
 (via (at 165.1 102.108) (size 0.8) (drill 0.4) (layers "F.Cu" "B.Cu") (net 1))
 (segment (start 174.752 84.836) (end 174.752 92.456) (width 0.25) (layer "B.Cu") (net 1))
 (segment (start 174.752 92.456) (end 165.1 102.108) (width 0.25) (layer "B.Cu") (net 1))
 (segment (start 174.859 81.427) (end 174.752 81.534) (width 0.25) (layer "F.Cu") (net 4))
 (segment (start 151.638 106.274) (end 164.979594 106.274) (width 0.25) (layer "F.Cu") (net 4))
 (segment (start 166.525 104.728594) (end 166.525 101.315) (width 0.25) (layer "F.Cu") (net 4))
 (segment (start 165.619 99.371) (end 165.619 93.008) (width 0.25) (layer "F.Cu") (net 4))
 (segment (start 158.496 84.6435) (end 159.5735 84.6435) (width 0.25) (layer "F.Cu") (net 4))
 (segment (start 165.1 99.89) (end 165.619 99.371) (width 0.25) (layer "F.Cu") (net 4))
 (segment (start 165.608 90.678) (end 165.608 92.997) (width 0.25) (layer "F.Cu") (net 4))
 (segment (start 166.525 101.315) (end 165.1 99.89) (width 0.25) (layer "F.Cu") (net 4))
 (segment (start 175.26 104.14) (end 169.35 104.14) (width 0.25) (layer "F.Cu") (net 4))
 (segment (start 159.5735 84.6435) (end 165.608 90.678) (width 0.25) (layer "F.Cu") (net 4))
 (segment (start 165.608 92.997) (end 165.619 93.008) (width 0.25) (layer "F.Cu") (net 4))
 (segment (start 164.979594 106.274) (end 166.525 104.728594) (width 0.25) (layer "F.Cu") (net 4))
 (segment (start 169.35 104.14) (end 165.1 99.89) (width 0.25) (layer "F.Cu") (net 4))
 (segment (start 176.276 81.427) (end 174.859 81.427) (width 0.25) (layer "F.Cu") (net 4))
 (via (at 174.752 81.534) (size 0.8) (drill 0.4) (layers "F.Cu" "B.Cu") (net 4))
 (via (at 165.608 90.678) (size 0.8) (drill 0.4) (layers "F.Cu" "B.Cu") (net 4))
 (segment (start 174.752 81.534) (end 165.608 90.678) (width 0.25) (layer "B.Cu") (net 4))
 (segment (start 161.2645 81.28) (end 159.0635 81.28) (width 0.25) (layer "F.Cu") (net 15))
 (segment (start 159.0635 81.28) (end 158.496 80.7125) (width 0.25) (layer "F.Cu") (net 15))
 (segment (start 171.469 86.71762) (end 171.469 85.808) (width 0.25) (layer "F.Cu") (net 16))
 (segment (start 179.73138 94.98) (end 171.469 86.71762) (width 0.25) (layer "F.Cu") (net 16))
 (segment (start 185.018 94.98) (end 179.73138 94.98) (width 0.25) (layer "F.Cu") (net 16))
 (segment (start 185.018 92.98) (end 179.291 92.98) (width 0.25) (layer "F.Cu") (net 17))
 (segment (start 179.291 92.98) (end 172.119 85.808) (width 0.25) (layer "F.Cu") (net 17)))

